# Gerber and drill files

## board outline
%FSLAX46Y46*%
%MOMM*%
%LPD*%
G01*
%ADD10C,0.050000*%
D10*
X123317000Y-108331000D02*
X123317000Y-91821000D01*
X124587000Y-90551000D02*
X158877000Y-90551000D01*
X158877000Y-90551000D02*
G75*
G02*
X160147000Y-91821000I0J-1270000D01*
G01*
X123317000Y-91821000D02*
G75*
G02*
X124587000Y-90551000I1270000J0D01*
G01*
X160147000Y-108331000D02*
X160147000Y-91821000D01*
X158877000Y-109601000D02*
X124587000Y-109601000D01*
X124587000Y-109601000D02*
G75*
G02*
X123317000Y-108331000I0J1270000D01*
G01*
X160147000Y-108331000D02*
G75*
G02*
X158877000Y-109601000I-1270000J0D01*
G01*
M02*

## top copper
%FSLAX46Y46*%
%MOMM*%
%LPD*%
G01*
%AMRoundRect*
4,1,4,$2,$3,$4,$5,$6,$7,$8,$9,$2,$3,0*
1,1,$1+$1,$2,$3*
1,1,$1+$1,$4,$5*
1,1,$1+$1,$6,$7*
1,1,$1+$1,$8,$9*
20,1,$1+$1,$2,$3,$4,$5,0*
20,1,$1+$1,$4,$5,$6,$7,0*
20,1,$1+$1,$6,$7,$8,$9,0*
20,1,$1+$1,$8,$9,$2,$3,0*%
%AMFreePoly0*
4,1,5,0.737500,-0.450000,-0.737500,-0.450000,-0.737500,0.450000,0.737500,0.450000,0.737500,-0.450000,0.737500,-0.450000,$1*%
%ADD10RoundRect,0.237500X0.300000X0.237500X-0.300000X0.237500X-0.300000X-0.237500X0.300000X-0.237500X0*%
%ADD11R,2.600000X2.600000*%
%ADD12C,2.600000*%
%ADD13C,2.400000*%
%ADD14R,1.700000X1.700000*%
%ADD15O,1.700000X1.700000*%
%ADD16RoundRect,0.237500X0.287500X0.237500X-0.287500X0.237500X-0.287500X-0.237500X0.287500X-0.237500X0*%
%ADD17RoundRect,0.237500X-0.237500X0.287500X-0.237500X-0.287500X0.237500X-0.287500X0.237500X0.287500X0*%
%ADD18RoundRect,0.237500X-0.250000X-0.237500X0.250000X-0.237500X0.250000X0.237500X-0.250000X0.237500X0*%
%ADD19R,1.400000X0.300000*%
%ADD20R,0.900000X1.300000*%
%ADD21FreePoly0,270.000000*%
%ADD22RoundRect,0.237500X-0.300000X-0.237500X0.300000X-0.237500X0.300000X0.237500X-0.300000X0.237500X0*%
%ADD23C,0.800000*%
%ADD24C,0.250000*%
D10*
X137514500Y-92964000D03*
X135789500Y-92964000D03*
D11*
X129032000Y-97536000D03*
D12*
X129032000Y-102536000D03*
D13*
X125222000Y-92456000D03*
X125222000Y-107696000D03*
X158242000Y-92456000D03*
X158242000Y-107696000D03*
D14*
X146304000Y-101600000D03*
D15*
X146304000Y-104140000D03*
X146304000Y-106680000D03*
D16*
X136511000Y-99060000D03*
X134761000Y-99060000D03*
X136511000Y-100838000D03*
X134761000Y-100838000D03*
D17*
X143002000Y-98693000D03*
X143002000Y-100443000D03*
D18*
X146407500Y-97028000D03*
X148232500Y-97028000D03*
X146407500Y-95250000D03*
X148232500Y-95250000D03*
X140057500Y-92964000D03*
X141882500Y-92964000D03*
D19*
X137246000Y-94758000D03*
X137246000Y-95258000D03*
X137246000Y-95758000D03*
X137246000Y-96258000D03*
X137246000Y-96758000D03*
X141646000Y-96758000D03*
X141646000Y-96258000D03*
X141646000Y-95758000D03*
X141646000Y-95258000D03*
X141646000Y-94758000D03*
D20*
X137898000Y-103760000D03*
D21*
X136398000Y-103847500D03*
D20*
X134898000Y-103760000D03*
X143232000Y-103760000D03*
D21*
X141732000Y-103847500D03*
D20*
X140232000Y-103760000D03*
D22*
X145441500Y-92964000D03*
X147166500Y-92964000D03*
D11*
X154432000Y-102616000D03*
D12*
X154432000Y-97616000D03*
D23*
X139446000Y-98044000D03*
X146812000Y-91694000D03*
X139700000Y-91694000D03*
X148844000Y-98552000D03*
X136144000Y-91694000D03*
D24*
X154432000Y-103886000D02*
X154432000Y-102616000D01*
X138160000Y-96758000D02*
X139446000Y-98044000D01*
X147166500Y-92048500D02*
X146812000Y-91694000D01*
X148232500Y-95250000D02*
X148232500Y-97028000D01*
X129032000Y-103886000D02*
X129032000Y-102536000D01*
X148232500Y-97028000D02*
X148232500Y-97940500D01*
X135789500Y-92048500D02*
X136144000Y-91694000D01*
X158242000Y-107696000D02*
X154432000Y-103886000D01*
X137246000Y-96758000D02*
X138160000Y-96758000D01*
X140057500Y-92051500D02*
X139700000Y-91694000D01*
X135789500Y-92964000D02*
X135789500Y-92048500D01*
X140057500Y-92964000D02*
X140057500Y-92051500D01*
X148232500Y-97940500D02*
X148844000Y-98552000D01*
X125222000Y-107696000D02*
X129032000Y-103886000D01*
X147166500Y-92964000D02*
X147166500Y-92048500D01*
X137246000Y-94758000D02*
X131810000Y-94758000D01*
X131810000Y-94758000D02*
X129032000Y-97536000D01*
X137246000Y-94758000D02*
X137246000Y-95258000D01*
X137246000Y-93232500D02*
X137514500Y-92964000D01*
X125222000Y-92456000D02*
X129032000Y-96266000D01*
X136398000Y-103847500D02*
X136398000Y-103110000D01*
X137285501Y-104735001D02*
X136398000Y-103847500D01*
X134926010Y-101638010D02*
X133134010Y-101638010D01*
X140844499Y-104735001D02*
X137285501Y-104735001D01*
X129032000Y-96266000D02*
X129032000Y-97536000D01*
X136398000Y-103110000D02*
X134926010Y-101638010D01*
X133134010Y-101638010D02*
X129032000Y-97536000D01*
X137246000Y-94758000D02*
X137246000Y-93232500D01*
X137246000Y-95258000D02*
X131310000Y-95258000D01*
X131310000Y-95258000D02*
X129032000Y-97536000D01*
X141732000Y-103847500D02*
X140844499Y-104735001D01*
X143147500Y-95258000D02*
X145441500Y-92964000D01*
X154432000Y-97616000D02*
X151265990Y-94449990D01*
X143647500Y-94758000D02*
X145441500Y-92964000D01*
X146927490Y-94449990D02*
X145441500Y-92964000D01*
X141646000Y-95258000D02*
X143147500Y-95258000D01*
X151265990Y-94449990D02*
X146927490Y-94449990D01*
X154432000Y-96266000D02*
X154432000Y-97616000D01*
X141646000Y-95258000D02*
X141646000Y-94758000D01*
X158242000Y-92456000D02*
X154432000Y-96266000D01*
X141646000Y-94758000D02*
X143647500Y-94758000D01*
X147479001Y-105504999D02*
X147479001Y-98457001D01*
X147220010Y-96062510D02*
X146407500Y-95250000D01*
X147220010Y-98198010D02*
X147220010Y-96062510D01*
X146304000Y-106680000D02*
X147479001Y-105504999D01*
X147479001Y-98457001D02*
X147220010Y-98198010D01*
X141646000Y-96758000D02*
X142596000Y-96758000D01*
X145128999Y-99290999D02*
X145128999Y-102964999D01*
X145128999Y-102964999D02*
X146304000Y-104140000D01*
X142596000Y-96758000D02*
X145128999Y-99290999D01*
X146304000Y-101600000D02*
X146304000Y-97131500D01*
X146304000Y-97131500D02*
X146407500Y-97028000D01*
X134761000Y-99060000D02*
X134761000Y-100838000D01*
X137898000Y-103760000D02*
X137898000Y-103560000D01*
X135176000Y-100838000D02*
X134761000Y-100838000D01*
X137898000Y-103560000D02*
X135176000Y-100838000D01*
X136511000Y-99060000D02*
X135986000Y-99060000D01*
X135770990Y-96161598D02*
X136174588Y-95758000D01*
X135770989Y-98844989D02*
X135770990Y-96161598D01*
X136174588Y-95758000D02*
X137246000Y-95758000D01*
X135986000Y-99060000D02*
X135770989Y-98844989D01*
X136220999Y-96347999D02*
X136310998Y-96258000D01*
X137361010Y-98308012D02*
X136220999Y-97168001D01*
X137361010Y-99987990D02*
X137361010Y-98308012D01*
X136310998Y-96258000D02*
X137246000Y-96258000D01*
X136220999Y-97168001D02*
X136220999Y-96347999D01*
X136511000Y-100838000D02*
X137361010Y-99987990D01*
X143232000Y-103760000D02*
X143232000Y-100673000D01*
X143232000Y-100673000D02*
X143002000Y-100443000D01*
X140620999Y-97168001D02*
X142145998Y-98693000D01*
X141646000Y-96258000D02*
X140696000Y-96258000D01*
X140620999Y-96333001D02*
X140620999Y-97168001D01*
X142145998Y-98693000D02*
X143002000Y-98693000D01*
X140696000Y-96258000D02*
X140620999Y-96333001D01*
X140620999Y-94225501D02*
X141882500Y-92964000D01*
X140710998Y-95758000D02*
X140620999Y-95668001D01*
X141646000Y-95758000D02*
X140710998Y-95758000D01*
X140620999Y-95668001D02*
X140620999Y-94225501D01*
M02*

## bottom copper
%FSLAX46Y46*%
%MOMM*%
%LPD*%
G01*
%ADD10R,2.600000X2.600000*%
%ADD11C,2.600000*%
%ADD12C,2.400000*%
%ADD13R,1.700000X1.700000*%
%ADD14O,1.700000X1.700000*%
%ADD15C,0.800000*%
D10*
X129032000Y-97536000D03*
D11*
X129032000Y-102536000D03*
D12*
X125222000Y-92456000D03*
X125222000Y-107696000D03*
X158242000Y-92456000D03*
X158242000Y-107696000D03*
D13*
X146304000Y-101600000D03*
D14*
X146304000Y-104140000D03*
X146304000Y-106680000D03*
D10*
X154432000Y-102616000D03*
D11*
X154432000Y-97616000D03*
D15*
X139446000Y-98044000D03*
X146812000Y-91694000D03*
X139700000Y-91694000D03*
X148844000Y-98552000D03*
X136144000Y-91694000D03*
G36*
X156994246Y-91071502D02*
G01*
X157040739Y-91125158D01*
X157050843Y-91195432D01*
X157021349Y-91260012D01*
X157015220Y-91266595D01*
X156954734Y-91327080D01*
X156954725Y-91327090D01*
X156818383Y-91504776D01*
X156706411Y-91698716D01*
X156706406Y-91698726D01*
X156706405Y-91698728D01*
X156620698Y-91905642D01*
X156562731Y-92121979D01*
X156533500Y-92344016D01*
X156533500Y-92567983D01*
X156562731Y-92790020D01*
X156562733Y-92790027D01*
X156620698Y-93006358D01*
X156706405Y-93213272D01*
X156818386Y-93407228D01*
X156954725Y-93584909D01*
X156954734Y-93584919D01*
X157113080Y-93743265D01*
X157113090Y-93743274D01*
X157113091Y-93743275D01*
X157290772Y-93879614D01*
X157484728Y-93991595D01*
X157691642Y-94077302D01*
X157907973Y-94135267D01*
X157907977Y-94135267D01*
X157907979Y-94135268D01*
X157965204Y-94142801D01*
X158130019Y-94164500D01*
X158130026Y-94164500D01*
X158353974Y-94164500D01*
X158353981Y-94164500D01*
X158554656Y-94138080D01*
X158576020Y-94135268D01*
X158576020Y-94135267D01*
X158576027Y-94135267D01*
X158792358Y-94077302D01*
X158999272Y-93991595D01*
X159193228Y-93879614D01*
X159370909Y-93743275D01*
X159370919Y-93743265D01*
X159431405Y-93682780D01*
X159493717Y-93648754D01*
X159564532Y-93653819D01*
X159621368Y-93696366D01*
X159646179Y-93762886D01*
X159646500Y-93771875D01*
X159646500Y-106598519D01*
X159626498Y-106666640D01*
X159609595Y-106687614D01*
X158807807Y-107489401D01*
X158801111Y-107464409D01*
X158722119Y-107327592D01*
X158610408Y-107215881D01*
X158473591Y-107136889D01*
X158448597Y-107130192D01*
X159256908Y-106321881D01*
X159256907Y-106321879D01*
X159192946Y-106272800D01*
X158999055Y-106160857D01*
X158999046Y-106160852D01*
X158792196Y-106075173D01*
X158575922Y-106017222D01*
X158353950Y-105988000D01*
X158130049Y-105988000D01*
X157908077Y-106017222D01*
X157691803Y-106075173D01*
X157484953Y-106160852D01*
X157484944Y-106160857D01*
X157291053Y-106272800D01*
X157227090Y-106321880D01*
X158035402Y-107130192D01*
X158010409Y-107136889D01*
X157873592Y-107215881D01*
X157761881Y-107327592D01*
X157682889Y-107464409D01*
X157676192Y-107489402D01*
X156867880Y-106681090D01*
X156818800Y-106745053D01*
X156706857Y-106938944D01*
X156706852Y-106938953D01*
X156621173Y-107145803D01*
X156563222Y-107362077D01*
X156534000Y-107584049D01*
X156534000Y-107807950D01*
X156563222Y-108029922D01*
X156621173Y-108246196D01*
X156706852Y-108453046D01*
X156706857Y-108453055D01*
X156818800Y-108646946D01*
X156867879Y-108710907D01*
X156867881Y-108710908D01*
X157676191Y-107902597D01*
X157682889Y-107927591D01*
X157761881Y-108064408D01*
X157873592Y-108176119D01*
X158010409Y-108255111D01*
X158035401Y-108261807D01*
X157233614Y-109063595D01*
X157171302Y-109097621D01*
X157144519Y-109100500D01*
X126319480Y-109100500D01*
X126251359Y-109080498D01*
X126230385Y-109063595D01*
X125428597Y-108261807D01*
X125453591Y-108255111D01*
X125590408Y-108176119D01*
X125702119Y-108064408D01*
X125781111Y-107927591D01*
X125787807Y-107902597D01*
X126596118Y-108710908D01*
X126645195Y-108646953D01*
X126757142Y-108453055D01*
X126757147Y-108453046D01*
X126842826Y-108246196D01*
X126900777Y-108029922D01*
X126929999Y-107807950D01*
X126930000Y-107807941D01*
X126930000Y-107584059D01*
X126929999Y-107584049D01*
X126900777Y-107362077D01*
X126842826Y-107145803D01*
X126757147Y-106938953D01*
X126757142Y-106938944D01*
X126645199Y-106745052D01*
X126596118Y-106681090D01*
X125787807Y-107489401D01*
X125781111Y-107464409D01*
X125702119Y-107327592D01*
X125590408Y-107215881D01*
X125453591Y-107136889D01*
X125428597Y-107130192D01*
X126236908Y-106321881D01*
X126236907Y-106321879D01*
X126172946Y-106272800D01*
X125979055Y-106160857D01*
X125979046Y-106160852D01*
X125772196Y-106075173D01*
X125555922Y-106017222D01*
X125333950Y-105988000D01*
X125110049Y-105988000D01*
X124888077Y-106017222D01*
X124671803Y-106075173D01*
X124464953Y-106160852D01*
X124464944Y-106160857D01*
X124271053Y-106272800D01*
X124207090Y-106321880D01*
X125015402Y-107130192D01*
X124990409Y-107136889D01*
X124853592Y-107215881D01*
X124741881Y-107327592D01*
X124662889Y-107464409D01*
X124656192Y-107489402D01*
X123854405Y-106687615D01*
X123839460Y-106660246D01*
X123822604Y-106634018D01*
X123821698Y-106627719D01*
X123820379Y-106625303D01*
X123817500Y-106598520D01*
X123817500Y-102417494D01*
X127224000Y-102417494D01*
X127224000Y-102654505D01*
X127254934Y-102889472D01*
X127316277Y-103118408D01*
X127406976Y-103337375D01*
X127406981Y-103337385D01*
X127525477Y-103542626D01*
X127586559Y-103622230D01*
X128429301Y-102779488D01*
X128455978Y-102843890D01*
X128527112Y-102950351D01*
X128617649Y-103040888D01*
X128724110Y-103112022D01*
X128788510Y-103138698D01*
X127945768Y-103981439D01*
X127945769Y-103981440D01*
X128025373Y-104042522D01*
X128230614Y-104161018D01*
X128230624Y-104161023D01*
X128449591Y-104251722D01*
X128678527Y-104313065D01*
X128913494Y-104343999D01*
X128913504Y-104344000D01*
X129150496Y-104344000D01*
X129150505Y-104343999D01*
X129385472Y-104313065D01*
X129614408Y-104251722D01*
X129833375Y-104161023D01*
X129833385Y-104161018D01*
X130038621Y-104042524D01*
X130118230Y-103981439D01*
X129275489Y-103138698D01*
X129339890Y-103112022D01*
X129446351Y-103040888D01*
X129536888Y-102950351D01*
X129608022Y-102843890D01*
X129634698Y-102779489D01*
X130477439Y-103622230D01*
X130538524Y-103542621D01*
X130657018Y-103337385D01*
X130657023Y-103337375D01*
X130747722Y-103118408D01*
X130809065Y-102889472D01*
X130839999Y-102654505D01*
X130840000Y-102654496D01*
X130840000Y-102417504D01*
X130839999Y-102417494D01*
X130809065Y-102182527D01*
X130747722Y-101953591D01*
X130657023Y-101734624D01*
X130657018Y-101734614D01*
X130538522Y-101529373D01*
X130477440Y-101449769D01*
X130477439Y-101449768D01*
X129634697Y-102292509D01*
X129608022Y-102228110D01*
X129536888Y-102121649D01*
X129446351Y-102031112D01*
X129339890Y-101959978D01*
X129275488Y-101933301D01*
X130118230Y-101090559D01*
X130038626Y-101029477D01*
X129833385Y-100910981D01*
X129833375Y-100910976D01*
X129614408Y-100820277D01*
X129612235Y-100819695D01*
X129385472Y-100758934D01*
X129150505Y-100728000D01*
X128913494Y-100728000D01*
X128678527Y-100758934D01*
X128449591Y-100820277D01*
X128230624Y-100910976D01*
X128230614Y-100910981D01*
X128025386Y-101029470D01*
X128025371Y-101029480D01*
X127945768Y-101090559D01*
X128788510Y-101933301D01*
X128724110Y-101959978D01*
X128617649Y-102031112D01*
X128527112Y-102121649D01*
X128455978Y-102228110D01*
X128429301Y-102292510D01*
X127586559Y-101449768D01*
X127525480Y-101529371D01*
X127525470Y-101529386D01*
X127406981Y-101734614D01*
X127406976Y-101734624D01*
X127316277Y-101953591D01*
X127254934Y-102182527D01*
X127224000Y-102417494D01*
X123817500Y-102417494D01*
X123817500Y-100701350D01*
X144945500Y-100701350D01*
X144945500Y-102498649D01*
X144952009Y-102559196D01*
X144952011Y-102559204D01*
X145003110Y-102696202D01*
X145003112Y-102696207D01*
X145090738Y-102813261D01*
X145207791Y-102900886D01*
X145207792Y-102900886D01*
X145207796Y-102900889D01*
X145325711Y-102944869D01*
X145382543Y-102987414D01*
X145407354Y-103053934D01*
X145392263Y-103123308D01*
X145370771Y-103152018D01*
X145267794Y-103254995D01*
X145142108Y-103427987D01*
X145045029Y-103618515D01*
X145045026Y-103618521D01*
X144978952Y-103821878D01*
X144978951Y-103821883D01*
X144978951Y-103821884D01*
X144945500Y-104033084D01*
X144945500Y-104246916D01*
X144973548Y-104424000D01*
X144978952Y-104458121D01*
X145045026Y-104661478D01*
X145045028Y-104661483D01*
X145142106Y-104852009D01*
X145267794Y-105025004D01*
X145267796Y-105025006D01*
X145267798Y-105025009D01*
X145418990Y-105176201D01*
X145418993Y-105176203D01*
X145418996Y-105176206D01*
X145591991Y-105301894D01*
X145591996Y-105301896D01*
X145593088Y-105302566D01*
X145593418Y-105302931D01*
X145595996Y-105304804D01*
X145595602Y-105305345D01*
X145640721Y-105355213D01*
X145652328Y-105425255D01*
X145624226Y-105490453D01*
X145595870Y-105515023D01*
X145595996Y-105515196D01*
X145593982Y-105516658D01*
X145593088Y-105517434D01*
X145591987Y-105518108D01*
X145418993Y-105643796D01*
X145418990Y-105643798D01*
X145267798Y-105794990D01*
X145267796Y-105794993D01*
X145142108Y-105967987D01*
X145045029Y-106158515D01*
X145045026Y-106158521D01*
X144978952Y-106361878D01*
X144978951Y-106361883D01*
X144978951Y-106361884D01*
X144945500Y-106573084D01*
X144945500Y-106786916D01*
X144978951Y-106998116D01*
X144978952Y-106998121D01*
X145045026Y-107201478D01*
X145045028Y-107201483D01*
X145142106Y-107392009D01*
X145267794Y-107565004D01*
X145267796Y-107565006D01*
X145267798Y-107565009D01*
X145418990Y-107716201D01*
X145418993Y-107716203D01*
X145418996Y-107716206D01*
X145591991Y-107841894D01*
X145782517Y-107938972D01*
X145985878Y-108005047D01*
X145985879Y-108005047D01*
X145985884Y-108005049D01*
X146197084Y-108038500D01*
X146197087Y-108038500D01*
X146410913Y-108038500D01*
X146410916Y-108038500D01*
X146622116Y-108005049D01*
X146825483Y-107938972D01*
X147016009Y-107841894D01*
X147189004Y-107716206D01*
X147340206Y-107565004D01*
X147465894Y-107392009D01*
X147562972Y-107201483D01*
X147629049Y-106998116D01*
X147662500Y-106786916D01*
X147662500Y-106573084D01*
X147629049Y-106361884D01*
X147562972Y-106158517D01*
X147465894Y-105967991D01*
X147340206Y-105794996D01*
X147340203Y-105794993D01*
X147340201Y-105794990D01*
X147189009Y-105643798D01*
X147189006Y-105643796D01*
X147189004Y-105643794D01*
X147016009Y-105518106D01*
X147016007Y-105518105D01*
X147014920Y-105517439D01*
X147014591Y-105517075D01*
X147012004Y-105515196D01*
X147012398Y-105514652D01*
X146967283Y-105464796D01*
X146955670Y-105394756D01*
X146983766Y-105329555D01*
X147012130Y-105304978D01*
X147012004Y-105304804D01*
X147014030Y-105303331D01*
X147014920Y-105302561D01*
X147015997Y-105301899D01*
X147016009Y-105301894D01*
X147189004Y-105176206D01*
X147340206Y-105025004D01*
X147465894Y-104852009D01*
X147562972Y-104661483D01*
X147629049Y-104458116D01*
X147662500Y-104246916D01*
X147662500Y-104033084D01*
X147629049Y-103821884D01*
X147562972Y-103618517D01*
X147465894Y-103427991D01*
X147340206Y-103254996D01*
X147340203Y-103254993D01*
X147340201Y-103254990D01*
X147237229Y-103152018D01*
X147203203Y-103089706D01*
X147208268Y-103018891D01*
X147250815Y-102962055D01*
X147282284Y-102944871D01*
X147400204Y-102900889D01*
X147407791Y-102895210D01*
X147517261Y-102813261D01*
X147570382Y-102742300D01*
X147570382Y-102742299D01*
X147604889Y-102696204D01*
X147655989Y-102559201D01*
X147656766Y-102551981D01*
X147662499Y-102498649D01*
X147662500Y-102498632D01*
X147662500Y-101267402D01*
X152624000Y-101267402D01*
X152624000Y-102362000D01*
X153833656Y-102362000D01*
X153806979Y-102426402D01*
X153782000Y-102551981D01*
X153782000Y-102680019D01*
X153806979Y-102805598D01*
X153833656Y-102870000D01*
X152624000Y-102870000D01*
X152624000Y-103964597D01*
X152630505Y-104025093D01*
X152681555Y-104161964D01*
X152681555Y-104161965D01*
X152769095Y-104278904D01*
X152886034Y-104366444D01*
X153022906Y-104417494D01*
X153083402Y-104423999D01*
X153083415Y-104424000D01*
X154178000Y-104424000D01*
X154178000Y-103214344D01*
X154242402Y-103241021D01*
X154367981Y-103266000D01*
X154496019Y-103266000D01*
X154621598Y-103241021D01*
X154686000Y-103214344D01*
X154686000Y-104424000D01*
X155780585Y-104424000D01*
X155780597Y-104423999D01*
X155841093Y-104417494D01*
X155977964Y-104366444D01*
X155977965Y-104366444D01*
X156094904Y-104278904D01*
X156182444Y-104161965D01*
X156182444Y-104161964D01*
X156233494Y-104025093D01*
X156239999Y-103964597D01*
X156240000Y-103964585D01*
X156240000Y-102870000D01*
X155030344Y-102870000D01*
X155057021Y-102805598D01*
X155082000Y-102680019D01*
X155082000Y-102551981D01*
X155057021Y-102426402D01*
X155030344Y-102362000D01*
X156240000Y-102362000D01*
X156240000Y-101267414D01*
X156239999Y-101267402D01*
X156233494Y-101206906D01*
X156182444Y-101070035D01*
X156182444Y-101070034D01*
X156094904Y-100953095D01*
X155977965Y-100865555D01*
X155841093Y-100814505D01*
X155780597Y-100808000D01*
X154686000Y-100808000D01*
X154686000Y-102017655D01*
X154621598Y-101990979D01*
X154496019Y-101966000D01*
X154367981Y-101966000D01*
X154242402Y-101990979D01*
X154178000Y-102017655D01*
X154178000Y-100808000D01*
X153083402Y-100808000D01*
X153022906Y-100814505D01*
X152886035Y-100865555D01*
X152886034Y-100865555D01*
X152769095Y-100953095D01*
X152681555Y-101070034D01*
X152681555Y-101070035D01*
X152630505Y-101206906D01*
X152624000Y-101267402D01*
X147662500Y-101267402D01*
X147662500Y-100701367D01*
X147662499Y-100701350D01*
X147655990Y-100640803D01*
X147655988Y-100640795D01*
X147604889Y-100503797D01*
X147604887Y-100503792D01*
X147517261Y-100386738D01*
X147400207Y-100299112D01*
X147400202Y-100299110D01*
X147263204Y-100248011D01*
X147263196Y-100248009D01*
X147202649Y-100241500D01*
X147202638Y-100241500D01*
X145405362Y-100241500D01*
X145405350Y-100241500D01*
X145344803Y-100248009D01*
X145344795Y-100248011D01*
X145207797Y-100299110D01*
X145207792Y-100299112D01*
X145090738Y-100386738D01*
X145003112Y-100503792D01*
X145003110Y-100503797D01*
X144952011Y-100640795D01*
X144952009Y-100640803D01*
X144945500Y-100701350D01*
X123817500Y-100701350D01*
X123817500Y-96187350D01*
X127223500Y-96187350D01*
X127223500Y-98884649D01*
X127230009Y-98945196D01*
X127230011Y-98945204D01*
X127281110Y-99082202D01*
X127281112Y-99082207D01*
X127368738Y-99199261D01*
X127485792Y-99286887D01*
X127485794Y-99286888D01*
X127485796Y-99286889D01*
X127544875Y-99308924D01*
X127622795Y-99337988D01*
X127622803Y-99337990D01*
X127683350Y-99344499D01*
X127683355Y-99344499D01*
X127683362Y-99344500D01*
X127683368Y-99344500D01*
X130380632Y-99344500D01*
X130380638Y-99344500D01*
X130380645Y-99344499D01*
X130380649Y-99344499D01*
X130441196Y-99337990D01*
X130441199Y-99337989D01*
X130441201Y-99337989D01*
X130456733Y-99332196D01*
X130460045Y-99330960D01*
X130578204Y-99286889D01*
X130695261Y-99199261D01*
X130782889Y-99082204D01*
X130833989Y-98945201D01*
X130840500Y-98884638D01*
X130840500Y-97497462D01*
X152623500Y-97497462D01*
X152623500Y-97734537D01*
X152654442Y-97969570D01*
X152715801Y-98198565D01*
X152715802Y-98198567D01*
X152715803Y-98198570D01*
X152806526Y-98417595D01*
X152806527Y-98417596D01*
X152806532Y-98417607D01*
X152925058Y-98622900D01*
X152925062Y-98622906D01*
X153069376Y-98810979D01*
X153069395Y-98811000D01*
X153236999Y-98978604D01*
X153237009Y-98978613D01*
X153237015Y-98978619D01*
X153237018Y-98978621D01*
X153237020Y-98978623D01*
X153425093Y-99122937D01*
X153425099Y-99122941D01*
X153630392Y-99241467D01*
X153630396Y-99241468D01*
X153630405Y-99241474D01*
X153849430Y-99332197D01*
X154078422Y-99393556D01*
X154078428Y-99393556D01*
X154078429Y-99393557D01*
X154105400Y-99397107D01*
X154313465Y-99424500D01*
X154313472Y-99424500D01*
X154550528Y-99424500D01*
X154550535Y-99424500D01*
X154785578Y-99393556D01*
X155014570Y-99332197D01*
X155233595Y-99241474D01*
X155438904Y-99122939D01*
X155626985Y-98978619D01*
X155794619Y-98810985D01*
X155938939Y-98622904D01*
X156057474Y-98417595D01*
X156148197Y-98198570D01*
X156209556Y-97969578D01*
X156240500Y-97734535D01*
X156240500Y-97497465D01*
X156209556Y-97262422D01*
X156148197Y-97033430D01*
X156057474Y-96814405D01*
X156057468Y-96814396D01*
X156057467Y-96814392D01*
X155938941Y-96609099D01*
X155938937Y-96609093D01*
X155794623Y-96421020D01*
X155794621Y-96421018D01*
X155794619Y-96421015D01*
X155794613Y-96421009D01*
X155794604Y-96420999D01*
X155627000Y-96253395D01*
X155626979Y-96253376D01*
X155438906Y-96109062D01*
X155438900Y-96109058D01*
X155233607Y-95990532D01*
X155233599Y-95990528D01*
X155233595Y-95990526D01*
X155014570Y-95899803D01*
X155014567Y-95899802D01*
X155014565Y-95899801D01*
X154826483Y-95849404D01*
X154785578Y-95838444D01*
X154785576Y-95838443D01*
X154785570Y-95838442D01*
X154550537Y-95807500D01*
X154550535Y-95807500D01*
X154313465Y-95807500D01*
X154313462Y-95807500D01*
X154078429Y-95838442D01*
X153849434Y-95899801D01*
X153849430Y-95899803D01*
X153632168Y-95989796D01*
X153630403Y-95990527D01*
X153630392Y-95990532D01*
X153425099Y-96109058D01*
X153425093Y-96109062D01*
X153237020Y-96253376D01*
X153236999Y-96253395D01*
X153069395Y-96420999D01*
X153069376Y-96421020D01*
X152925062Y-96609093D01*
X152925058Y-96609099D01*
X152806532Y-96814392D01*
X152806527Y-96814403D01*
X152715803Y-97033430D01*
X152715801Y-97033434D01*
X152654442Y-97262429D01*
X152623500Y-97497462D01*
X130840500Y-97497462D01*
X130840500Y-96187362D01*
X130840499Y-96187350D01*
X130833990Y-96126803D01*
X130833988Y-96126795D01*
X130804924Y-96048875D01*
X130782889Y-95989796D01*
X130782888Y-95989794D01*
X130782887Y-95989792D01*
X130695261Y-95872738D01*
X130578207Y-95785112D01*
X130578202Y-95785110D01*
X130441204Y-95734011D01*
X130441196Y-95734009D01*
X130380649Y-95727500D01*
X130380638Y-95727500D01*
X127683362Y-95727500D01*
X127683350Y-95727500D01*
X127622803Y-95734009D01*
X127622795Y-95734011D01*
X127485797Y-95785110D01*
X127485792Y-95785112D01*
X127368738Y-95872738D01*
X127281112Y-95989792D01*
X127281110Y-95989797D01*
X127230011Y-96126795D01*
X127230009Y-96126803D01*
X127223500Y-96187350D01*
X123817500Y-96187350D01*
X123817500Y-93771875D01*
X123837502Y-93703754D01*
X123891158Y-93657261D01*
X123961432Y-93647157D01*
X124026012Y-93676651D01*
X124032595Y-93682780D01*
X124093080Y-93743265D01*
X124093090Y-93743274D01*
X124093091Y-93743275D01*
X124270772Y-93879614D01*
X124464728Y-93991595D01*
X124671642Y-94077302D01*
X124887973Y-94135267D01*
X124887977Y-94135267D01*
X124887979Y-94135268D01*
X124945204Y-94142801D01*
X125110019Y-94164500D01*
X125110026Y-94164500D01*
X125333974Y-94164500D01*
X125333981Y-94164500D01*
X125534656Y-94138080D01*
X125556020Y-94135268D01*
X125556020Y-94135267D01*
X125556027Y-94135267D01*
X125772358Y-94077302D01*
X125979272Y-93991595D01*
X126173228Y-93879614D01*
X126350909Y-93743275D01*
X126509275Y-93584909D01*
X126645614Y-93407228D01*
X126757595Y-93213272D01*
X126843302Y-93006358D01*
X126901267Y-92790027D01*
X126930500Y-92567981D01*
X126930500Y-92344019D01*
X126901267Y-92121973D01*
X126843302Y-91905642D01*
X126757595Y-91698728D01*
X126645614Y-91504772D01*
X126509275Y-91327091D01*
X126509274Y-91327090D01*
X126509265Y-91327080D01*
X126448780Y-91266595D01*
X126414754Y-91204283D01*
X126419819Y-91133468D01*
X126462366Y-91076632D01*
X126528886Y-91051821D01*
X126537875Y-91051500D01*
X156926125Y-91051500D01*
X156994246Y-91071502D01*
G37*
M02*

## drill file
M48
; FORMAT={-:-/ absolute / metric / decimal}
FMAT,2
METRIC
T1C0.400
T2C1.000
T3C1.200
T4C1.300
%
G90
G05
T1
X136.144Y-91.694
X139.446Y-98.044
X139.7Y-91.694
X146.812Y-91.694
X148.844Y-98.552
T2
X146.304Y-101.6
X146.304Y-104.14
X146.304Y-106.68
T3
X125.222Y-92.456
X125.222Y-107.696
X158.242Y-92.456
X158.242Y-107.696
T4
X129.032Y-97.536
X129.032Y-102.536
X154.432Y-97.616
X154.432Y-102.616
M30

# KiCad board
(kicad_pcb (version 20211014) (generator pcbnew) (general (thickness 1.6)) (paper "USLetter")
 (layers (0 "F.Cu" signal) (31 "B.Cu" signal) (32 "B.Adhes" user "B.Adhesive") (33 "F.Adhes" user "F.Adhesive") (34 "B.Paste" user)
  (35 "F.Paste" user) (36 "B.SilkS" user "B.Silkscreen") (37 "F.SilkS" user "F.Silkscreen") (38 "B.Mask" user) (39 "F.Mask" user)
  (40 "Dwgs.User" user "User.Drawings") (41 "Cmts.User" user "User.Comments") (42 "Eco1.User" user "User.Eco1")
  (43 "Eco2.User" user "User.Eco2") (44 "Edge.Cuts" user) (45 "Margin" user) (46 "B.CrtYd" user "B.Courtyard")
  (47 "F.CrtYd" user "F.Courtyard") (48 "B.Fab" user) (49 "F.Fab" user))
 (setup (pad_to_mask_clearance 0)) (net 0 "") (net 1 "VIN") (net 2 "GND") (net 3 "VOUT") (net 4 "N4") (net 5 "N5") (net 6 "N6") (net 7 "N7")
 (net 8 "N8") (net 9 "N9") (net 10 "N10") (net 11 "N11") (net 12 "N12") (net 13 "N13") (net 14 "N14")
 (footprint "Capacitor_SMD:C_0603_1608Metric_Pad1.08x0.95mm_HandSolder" (layer "F.Cu") (at 136.652 92.964 180)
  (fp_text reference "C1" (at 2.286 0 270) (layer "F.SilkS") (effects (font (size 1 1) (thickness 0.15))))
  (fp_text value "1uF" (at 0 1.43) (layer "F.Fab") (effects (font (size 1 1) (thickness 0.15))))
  (pad "1" smd roundrect locked (at -0.8625 0 180) (size 1.075 0.95) (layers "F.Cu" "F.Paste" "F.Mask") (roundrect_rratio 0.25)
   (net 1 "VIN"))
  (pad "2" smd roundrect locked (at 0.8625 0 180) (size 1.075 0.95) (layers "F.Cu" "F.Paste" "F.Mask") (roundrect_rratio 0.25) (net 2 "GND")))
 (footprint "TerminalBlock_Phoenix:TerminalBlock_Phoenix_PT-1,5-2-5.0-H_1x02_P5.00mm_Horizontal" (layer "F.Cu") (at 129.032 97.536 -90)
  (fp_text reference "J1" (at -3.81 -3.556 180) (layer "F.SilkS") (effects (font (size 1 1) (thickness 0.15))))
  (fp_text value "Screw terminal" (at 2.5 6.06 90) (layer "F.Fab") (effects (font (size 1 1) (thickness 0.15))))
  (pad "1" thru_hole rect locked (at 0 0 270) (size 2.6 2.6) (drill 1.3) (layers *.Cu *.Mask) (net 1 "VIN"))
  (pad "2" thru_hole circle locked (at 5 0 270) (size 2.6 2.6) (drill 1.3) (layers *.Cu *.Mask) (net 2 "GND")))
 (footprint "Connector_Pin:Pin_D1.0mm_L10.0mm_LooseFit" (layer "F.Cu") (at 125.222 92.456 90)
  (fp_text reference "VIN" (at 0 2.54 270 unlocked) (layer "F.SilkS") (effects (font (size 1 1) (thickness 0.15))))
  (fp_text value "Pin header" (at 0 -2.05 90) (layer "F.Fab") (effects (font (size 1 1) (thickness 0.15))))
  (pad "1" thru_hole circle locked (at 0 0 90) (size 2.4 2.4) (drill 1.2) (layers *.Cu *.Mask) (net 1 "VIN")))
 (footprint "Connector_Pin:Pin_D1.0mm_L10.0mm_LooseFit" (layer "F.Cu") (at 125.222 107.696 90)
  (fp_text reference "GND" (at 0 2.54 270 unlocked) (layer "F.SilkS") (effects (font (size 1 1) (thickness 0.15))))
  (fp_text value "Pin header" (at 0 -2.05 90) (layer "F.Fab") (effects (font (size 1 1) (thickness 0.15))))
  (pad "1" thru_hole circle locked (at 0 0 90) (size 2.4 2.4) (drill 1.2) (layers *.Cu *.Mask) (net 2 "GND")))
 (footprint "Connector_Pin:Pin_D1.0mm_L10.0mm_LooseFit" (layer "F.Cu") (at 158.242 92.456 -90)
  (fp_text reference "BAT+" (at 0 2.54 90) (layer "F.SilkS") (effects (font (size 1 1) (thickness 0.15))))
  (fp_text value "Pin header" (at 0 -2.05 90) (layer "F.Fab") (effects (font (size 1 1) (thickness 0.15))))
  (pad "1" thru_hole circle locked (at 0 0 270) (size 2.4 2.4) (drill 1.2) (layers *.Cu *.Mask) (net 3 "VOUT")))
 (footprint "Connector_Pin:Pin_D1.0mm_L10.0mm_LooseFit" (layer "F.Cu") (at 158.242 107.696 -90)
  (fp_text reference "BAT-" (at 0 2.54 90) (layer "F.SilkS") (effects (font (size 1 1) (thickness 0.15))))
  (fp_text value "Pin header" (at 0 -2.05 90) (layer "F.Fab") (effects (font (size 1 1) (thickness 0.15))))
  (pad "1" thru_hole circle locked (at 0 0 270) (size 2.4 2.4) (drill 1.2) (layers *.Cu *.Mask) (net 2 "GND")))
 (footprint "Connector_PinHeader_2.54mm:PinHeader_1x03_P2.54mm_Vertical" (layer "F.Cu") (at 146.304 101.6)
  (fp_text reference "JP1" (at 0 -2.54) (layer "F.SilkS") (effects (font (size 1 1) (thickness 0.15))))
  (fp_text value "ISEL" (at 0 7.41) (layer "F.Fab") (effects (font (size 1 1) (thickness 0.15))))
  (pad "1" thru_hole rect locked (at 0 0) (size 1.7 1.7) (drill 1) (layers *.Cu *.Mask) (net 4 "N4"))
  (pad "2" thru_hole oval locked (at 0 2.54) (size 1.7 1.7) (drill 1) (layers *.Cu *.Mask) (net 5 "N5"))
  (pad "3" thru_hole oval locked (at 0 5.08) (size 1.7 1.7) (drill 1) (layers *.Cu *.Mask) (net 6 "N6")))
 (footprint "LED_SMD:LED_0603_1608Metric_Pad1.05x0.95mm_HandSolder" (layer "F.Cu") (at 135.636 99.06 180)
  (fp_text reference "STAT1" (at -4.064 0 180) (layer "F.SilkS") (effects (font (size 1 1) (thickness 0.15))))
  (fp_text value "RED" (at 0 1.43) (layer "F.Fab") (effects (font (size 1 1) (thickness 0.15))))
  (pad "1" smd roundrect locked (at -0.875 0 180) (size 1.05 0.95) (layers "F.Cu" "F.Paste" "F.Mask") (roundrect_rratio 0.25) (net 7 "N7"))
  (pad "2" smd roundrect locked (at 0.875 0 180) (size 1.05 0.95) (layers "F.Cu" "F.Paste" "F.Mask") (roundrect_rratio 0.25) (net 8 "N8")))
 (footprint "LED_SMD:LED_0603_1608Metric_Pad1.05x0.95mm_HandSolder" (layer "F.Cu") (at 135.636 100.838 180)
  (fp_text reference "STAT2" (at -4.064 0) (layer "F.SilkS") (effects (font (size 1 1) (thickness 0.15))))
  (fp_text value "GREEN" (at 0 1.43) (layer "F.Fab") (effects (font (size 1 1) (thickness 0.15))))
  (pad "1" smd roundrect locked (at -0.875 0 180) (size 1.05 0.95) (layers "F.Cu" "F.Paste" "F.Mask") (roundrect_rratio 0.25) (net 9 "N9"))
  (pad "2" smd roundrect locked (at 0.875 0 180) (size 1.05 0.95) (layers "F.Cu" "F.Paste" "F.Mask") (roundrect_rratio 0.25) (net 8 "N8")))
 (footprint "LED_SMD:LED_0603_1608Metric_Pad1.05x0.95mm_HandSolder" (layer "F.Cu") (at 143.002 99.568 -90)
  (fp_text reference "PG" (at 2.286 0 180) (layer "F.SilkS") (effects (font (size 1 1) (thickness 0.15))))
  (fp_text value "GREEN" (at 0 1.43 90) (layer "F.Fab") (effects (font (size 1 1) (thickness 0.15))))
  (pad "1" smd roundrect locked (at -0.875 0 270) (size 1.05 0.95) (layers "F.Cu" "F.Paste" "F.Mask") (roundrect_rratio 0.25) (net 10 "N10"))
  (pad "2" smd roundrect locked (at 0.875 0 270) (size 1.05 0.95) (layers "F.Cu" "F.Paste" "F.Mask") (roundrect_rratio 0.25) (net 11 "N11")))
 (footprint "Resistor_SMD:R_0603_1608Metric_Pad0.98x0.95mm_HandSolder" (layer "F.Cu") (at 147.32 97.028)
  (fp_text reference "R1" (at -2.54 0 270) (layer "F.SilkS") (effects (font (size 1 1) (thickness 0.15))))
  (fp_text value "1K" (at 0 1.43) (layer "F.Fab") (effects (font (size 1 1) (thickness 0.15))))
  (pad "1" smd roundrect locked (at -0.9125 0) (size 0.975 0.95) (layers "F.Cu" "F.Paste" "F.Mask") (roundrect_rratio 0.25) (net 4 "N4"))
  (pad "2" smd roundrect locked (at 0.9125 0) (size 0.975 0.95) (layers "F.Cu" "F.Paste" "F.Mask") (roundrect_rratio 0.25) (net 2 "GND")))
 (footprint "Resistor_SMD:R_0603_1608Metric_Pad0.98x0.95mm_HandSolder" (layer "F.Cu") (at 147.32 95.25)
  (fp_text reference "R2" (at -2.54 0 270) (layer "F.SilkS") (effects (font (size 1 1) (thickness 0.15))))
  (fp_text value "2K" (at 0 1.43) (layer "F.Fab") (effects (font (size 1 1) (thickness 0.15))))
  (pad "1" smd roundrect locked (at -0.9125 0) (size 0.975 0.95) (layers "F.Cu" "F.Paste" "F.Mask") (roundrect_rratio 0.25) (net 6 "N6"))
  (pad "2" smd roundrect locked (at 0.9125 0) (size 0.975 0.95) (layers "F.Cu" "F.Paste" "F.Mask") (roundrect_rratio 0.25) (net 2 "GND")))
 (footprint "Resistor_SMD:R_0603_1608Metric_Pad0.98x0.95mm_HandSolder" (layer "F.Cu") (at 140.97 92.964)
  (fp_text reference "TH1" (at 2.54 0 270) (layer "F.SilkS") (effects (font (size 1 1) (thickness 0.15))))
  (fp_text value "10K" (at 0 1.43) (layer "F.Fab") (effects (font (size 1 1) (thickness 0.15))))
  (pad "1" smd roundrect locked (at -0.9125 0) (size 0.975 0.95) (layers "F.Cu" "F.Paste" "F.Mask") (roundrect_rratio 0.25) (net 2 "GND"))
  (pad "2" smd roundrect locked (at 0.9125 0) (size 0.975 0.95) (layers "F.Cu" "F.Paste" "F.Mask") (roundrect_rratio 0.25) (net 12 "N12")))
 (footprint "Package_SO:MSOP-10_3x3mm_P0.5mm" (layer "F.Cu") (at 139.446 95.758)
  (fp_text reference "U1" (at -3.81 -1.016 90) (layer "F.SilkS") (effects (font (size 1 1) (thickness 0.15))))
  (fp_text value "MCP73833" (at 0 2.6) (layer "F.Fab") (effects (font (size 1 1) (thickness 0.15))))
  (pad "1" smd rect locked (at -2.2 -1) (size 1.4 0.3) (layers "F.Cu" "F.Paste" "F.Mask") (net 1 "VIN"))
  (pad "2" smd rect locked (at -2.2 -0.5) (size 1.4 0.3) (layers "F.Cu" "F.Paste" "F.Mask") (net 1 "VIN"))
  (pad "3" smd rect locked (at -2.2 0) (size 1.4 0.3) (layers "F.Cu" "F.Paste" "F.Mask") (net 7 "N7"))
  (pad "4" smd rect locked (at -2.2 0.5) (size 1.4 0.3) (layers "F.Cu" "F.Paste" "F.Mask") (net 9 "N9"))
  (pad "5" smd rect locked (at -2.2 1) (size 1.4 0.3) (layers "F.Cu" "F.Paste" "F.Mask") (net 2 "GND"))
  (pad "6" smd rect locked (at 2.2 1) (size 1.4 0.3) (layers "F.Cu" "F.Paste" "F.Mask") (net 5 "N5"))
  (pad "7" smd rect locked (at 2.2 0.5) (size 1.4 0.3) (layers "F.Cu" "F.Paste" "F.Mask") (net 10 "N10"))
  (pad "8" smd rect locked (at 2.2 0) (size 1.4 0.3) (layers "F.Cu" "F.Paste" "F.Mask") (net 12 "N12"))
  (pad "9" smd rect locked (at 2.2 -0.5) (size 1.4 0.3) (layers "F.Cu" "F.Paste" "F.Mask") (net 3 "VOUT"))
  (pad "10" smd rect locked (at 2.2 -1) (size 1.4 0.3) (layers "F.Cu" "F.Paste" "F.Mask") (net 3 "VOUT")))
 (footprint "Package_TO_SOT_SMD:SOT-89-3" (layer "F.Cu") (at 136.398 105.41 -90)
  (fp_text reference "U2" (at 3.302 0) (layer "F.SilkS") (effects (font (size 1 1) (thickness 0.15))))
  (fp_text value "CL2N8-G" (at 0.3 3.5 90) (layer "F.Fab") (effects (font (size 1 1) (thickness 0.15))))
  (pad "1" smd rect locked (at -1.65 -1.5 270) (size 1.3 0.9) (layers "F.Cu" "F.Paste" "F.Mask") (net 8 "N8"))
  (pad "2" smd custom locked (at -1.5625 0 270) (size 1.475 0.9) (layers "F.Cu" "F.Paste" "F.Mask") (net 1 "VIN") (zone_connect 2)
   (options (clearance outline) (anchor rect)) (primitives))
  (pad "3" smd rect locked (at -1.65 1.5 270) (size 1.3 0.9) (layers "F.Cu" "F.Paste" "F.Mask") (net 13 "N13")))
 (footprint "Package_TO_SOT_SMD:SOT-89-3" (layer "F.Cu") (at 141.732 105.41 -90)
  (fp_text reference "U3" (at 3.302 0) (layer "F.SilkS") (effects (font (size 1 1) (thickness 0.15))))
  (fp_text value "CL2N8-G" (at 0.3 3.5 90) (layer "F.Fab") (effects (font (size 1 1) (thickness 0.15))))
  (pad "1" smd rect locked (at -1.65 -1.5 270) (size 1.3 0.9) (layers "F.Cu" "F.Paste" "F.Mask") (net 11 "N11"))
  (pad "2" smd custom locked (at -1.5625 0 270) (size 1.475 0.9) (layers "F.Cu" "F.Paste" "F.Mask") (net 1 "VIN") (zone_connect 2)
   (options (clearance outline) (anchor rect)) (primitives))
  (pad "3" smd rect locked (at -1.65 1.5 270) (size 1.3 0.9) (layers "F.Cu" "F.Paste" "F.Mask") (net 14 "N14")))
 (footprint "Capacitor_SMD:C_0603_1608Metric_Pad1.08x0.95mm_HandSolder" (layer "F.Cu") (at 146.304 92.964)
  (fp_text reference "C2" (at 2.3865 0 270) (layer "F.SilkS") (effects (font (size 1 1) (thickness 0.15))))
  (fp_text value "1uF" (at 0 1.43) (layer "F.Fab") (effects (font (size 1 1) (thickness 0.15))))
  (pad "1" smd roundrect locked (at -0.8625 0) (size 1.075 0.95) (layers "F.Cu" "F.Paste" "F.Mask") (roundrect_rratio 0.25) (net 3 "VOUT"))
  (pad "2" smd roundrect locked (at 0.8625 0) (size 1.075 0.95) (layers "F.Cu" "F.Paste" "F.Mask") (roundrect_rratio 0.25) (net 2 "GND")))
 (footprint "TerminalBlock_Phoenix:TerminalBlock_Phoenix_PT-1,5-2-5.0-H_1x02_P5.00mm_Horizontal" (layer "F.Cu") (at 154.432 102.616 90)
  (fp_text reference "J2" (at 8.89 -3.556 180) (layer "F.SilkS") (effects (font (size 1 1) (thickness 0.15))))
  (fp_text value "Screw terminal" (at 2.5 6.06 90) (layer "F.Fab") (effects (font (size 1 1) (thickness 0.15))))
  (pad "1" thru_hole rect locked (at 0 0 90) (size 2.6 2.6) (drill 1.3) (layers *.Cu *.Mask) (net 2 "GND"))
  (pad "2" thru_hole circle locked (at 5 0 90) (size 2.6 2.6) (drill 1.3) (layers *.Cu *.Mask) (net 3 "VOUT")))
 (gr_line (start 123.317 108.331) (end 123.317 91.821) (layer "Edge.Cuts") (width 0.05))
 (gr_line (start 124.587 90.551) (end 158.877 90.551) (layer "Edge.Cuts") (width 0.05))
 (gr_arc (start 158.877 90.551) (mid 159.775026 90.922974) (end 160.147 91.821) (layer "Edge.Cuts") (width 0.05))
 (gr_arc (start 123.317 91.821) (mid 123.688974 90.922974) (end 124.587 90.551) (layer "Edge.Cuts") (width 0.05))
 (gr_line (start 160.147 108.331) (end 160.147 91.821) (layer "Edge.Cuts") (width 0.05))
 (gr_line (start 158.877 109.601) (end 124.587 109.601) (layer "Edge.Cuts") (width 0.05))
 (gr_arc (start 124.587 109.601) (mid 123.688974 109.229026) (end 123.317 108.331) (layer "Edge.Cuts") (width 0.05))
 (gr_arc (start 160.147 108.331) (mid 159.775026 109.229026) (end 158.877 109.601) (layer "Edge.Cuts") (width 0.05))
 (segment (start 154.432 103.886) (end 154.432 102.616) (width 0.25) (layer "F.Cu") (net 2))
 (segment (start 138.16 96.758) (end 139.446 98.044) (width 0.25) (layer "F.Cu") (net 2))
 (segment (start 147.1665 92.0485) (end 146.812 91.694) (width 0.25) (layer "F.Cu") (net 2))
 (segment (start 148.2325 95.25) (end 148.2325 97.028) (width 0.25) (layer "F.Cu") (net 2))
 (segment (start 129.032 103.886) (end 129.032 102.536) (width 0.25) (layer "F.Cu") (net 2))
 (segment (start 148.2325 97.028) (end 148.2325 97.9405) (width 0.25) (layer "F.Cu") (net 2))
 (segment (start 135.7895 92.0485) (end 136.144 91.694) (width 0.25) (layer "F.Cu") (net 2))
 (segment (start 158.242 107.696) (end 154.432 103.886) (width 0.25) (layer "F.Cu") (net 2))
 (segment (start 137.246 96.758) (end 138.16 96.758) (width 0.25) (layer "F.Cu") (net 2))
 (segment (start 140.0575 92.0515) (end 139.7 91.694) (width 0.25) (layer "F.Cu") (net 2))
 (segment (start 135.7895 92.964) (end 135.7895 92.0485) (width 0.25) (layer "F.Cu") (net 2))
 (segment (start 140.0575 92.964) (end 140.0575 92.0515) (width 0.25) (layer "F.Cu") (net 2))
 (segment (start 148.2325 97.9405) (end 148.844 98.552) (width 0.25) (layer "F.Cu") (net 2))
 (segment (start 125.222 107.696) (end 129.032 103.886) (width 0.25) (layer "F.Cu") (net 2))
 (segment (start 147.1665 92.964) (end 147.1665 92.0485) (width 0.25) (layer "F.Cu") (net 2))
 (via (at 139.446 98.044) (size 0.8) (drill 0.4) (layers "F.Cu" "B.Cu") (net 2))
 (via (at 146.812 91.694) (size 0.8) (drill 0.4) (layers "F.Cu" "B.Cu") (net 2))
 (via (at 139.7 91.694) (size 0.8) (drill 0.4) (layers "F.Cu" "B.Cu") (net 2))
 (via (at 148.844 98.552) (size 0.8) (drill 0.4) (layers "F.Cu" "B.Cu") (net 2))
 (via (at 136.144 91.694) (size 0.8) (drill 0.4) (layers "F.Cu" "B.Cu") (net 2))
 (segment (start 137.246 94.758) (end 131.81 94.758) (width 0.25) (layer "F.Cu") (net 1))
 (segment (start 131.81 94.758) (end 129.032 97.536) (width 0.25) (layer "F.Cu") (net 1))
 (segment (start 137.246 94.758) (end 137.246 95.258) (width 0.25) (layer "F.Cu") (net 1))
 (segment (start 137.246 93.2325) (end 137.5145 92.964) (width 0.25) (layer "F.Cu") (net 1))
 (segment (start 125.222 92.456) (end 129.032 96.266) (width 0.25) (layer "F.Cu") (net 1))
 (segment (start 136.398 103.8475) (end 136.398 103.11) (width 0.25) (layer "F.Cu") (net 1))
 (segment (start 137.285501 104.735001) (end 136.398 103.8475) (width 0.25) (layer "F.Cu") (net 1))
 (segment (start 134.92601 101.63801) (end 133.13401 101.63801) (width 0.25) (layer "F.Cu") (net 1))
 (segment (start 140.844499 104.735001) (end 137.285501 104.735001) (width 0.25) (layer "F.Cu") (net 1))
 (segment (start 129.032 96.266) (end 129.032 97.536) (width 0.25) (layer "F.Cu") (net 1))
 (segment (start 136.398 103.11) (end 134.92601 101.63801) (width 0.25) (layer "F.Cu") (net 1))
 (segment (start 133.13401 101.63801) (end 129.032 97.536) (width 0.25) (layer "F.Cu") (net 1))
 (segment (start 137.246 94.758) (end 137.246 93.2325) (width 0.25) (layer "F.Cu") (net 1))
 (segment (start 137.246 95.258) (end 131.31 95.258) (width 0.25) (layer "F.Cu") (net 1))
 (segment (start 131.31 95.258) (end 129.032 97.536) (width 0.25) (layer "F.Cu") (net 1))
 (segment (start 141.732 103.8475) (end 140.844499 104.735001) (width 0.25) (layer "F.Cu") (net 1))
 (segment (start 143.1475 95.258) (end 145.4415 92.964) (width 0.25) (layer "F.Cu") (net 3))
 (segment (start 154.432 97.616) (end 151.26599 94.44999) (width 0.25) (layer "F.Cu") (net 3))
 (segment (start 143.6475 94.758) (end 145.4415 92.964) (width 0.25) (layer "F.Cu") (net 3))
 (segment (start 146.92749 94.44999) (end 145.4415 92.964) (width 0.25) (layer "F.Cu") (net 3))
 (segment (start 141.646 95.258) (end 143.1475 95.258) (width 0.25) (layer "F.Cu") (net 3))
 (segment (start 151.26599 94.44999) (end 146.92749 94.44999) (width 0.25) (layer "F.Cu") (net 3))
 (segment (start 154.432 96.266) (end 154.432 97.616) (width 0.25) (layer "F.Cu") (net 3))
 (segment (start 141.646 95.258) (end 141.646 94.758) (width 0.25) (layer "F.Cu") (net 3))
 (segment (start 158.242 92.456) (end 154.432 96.266) (width 0.25) (layer "F.Cu") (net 3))
 (segment (start 141.646 94.758) (end 143.6475 94.758) (width 0.25) (layer "F.Cu") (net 3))
 (segment (start 147.479001 105.504999) (end 147.479001 98.457001) (width 0.25) (layer "F.Cu") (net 6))
 (segment (start 147.22001 96.06251) (end 146.4075 95.25) (width 0.25) (layer "F.Cu") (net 6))
 (segment (start 147.22001 98.19801) (end 147.22001 96.06251) (width 0.25) (layer "F.Cu") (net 6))
 (segment (start 146.304 106.68) (end 147.479001 105.504999) (width 0.25) (layer "F.Cu") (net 6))
 (segment (start 147.479001 98.457001) (end 147.22001 98.19801) (width 0.25) (layer "F.Cu") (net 6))
 (segment (start 141.646 96.758) (end 142.596 96.758) (width 0.25) (layer "F.Cu") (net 5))
 (segment (start 145.128999 99.290999) (end 145.128999 102.964999) (width 0.25) (layer "F.Cu") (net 5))
 (segment (start 145.128999 102.964999) (end 146.304 104.14) (width 0.25) (layer "F.Cu") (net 5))
 (segment (start 142.596 96.758) (end 145.128999 99.290999) (width 0.25) (layer "F.Cu") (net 5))
 (segment (start 146.304 101.6) (end 146.304 97.1315) (width 0.25) (layer "F.Cu") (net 4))
 (segment (start 146.304 97.1315) (end 146.4075 97.028) (width 0.25) (layer "F.Cu") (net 4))
 (segment (start 134.761 99.06) (end 134.761 100.838) (width 0.25) (layer "F.Cu") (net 8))
 (segment (start 137.898 103.76) (end 137.898 103.56) (width 0.25) (layer "F.Cu") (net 8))
 (segment (start 135.176 100.838) (end 134.761 100.838) (width 0.25) (layer "F.Cu") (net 8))
 (segment (start 137.898 103.56) (end 135.176 100.838) (width 0.25) (layer "F.Cu") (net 8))
 (segment (start 136.511 99.06) (end 135.986 99.06) (width 0.25) (layer "F.Cu") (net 7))
 (segment (start 135.77099 96.161598) (end 136.174588 95.758) (width 0.25) (layer "F.Cu") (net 7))
 (segment (start 135.770989 98.844989) (end 135.77099 96.161598) (width 0.25) (layer "F.Cu") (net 7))
 (segment (start 136.174588 95.758) (end 137.246 95.758) (width 0.25) (layer "F.Cu") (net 7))
 (segment (start 135.986 99.06) (end 135.770989 98.844989) (width 0.25) (layer "F.Cu") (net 7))
 (segment (start 136.220999 96.347999) (end 136.310998 96.258) (width 0.25) (layer "F.Cu") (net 9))
 (segment (start 137.36101 98.308012) (end 136.220999 97.168001) (width 0.25) (layer "F.Cu") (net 9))
 (segment (start 137.36101 99.98799) (end 137.36101 98.308012) (width 0.25) (layer "F.Cu") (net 9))
 (segment (start 136.310998 96.258) (end 137.246 96.258) (width 0.25) (layer "F.Cu") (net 9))
 (segment (start 136.220999 97.168001) (end 136.220999 96.347999) (width 0.25) (layer "F.Cu") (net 9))
 (segment (start 136.511 100.838) (end 137.36101 99.98799) (width 0.25) (layer "F.Cu") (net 9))
 (segment (start 143.232 103.76) (end 143.232 100.673) (width 0.25) (layer "F.Cu") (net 11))
 (segment (start 143.232 100.673) (end 143.002 100.443) (width 0.25) (layer "F.Cu") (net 11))
 (segment (start 140.620999 97.168001) (end 142.145998 98.693) (width 0.25) (layer "F.Cu") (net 10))
 (segment (start 141.646 96.258) (end 140.696 96.258) (width 0.25) (layer "F.Cu") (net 10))
 (segment (start 140.620999 96.333001) (end 140.620999 97.168001) (width 0.25) (layer "F.Cu") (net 10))
 (segment (start 142.145998 98.693) (end 143.002 98.693) (width 0.25) (layer "F.Cu") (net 10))
 (segment (start 140.696 96.258) (end 140.620999 96.333001) (width 0.25) (layer "F.Cu") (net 10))
 (segment (start 140.620999 94.225501) (end 141.8825 92.964) (width 0.25) (layer "F.Cu") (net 12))
 (segment (start 140.710998 95.758) (end 140.620999 95.668001) (width 0.25) (layer "F.Cu") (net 12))
 (segment (start 141.646 95.758) (end 140.710998 95.758) (width 0.25) (layer "F.Cu") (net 12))
 (segment (start 140.620999 95.668001) (end 140.620999 94.225501) (width 0.25) (layer "F.Cu") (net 12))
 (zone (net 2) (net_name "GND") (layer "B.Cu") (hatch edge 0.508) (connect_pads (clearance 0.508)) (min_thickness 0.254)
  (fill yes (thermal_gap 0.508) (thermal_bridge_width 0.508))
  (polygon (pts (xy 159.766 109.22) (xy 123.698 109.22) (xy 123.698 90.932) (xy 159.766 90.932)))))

